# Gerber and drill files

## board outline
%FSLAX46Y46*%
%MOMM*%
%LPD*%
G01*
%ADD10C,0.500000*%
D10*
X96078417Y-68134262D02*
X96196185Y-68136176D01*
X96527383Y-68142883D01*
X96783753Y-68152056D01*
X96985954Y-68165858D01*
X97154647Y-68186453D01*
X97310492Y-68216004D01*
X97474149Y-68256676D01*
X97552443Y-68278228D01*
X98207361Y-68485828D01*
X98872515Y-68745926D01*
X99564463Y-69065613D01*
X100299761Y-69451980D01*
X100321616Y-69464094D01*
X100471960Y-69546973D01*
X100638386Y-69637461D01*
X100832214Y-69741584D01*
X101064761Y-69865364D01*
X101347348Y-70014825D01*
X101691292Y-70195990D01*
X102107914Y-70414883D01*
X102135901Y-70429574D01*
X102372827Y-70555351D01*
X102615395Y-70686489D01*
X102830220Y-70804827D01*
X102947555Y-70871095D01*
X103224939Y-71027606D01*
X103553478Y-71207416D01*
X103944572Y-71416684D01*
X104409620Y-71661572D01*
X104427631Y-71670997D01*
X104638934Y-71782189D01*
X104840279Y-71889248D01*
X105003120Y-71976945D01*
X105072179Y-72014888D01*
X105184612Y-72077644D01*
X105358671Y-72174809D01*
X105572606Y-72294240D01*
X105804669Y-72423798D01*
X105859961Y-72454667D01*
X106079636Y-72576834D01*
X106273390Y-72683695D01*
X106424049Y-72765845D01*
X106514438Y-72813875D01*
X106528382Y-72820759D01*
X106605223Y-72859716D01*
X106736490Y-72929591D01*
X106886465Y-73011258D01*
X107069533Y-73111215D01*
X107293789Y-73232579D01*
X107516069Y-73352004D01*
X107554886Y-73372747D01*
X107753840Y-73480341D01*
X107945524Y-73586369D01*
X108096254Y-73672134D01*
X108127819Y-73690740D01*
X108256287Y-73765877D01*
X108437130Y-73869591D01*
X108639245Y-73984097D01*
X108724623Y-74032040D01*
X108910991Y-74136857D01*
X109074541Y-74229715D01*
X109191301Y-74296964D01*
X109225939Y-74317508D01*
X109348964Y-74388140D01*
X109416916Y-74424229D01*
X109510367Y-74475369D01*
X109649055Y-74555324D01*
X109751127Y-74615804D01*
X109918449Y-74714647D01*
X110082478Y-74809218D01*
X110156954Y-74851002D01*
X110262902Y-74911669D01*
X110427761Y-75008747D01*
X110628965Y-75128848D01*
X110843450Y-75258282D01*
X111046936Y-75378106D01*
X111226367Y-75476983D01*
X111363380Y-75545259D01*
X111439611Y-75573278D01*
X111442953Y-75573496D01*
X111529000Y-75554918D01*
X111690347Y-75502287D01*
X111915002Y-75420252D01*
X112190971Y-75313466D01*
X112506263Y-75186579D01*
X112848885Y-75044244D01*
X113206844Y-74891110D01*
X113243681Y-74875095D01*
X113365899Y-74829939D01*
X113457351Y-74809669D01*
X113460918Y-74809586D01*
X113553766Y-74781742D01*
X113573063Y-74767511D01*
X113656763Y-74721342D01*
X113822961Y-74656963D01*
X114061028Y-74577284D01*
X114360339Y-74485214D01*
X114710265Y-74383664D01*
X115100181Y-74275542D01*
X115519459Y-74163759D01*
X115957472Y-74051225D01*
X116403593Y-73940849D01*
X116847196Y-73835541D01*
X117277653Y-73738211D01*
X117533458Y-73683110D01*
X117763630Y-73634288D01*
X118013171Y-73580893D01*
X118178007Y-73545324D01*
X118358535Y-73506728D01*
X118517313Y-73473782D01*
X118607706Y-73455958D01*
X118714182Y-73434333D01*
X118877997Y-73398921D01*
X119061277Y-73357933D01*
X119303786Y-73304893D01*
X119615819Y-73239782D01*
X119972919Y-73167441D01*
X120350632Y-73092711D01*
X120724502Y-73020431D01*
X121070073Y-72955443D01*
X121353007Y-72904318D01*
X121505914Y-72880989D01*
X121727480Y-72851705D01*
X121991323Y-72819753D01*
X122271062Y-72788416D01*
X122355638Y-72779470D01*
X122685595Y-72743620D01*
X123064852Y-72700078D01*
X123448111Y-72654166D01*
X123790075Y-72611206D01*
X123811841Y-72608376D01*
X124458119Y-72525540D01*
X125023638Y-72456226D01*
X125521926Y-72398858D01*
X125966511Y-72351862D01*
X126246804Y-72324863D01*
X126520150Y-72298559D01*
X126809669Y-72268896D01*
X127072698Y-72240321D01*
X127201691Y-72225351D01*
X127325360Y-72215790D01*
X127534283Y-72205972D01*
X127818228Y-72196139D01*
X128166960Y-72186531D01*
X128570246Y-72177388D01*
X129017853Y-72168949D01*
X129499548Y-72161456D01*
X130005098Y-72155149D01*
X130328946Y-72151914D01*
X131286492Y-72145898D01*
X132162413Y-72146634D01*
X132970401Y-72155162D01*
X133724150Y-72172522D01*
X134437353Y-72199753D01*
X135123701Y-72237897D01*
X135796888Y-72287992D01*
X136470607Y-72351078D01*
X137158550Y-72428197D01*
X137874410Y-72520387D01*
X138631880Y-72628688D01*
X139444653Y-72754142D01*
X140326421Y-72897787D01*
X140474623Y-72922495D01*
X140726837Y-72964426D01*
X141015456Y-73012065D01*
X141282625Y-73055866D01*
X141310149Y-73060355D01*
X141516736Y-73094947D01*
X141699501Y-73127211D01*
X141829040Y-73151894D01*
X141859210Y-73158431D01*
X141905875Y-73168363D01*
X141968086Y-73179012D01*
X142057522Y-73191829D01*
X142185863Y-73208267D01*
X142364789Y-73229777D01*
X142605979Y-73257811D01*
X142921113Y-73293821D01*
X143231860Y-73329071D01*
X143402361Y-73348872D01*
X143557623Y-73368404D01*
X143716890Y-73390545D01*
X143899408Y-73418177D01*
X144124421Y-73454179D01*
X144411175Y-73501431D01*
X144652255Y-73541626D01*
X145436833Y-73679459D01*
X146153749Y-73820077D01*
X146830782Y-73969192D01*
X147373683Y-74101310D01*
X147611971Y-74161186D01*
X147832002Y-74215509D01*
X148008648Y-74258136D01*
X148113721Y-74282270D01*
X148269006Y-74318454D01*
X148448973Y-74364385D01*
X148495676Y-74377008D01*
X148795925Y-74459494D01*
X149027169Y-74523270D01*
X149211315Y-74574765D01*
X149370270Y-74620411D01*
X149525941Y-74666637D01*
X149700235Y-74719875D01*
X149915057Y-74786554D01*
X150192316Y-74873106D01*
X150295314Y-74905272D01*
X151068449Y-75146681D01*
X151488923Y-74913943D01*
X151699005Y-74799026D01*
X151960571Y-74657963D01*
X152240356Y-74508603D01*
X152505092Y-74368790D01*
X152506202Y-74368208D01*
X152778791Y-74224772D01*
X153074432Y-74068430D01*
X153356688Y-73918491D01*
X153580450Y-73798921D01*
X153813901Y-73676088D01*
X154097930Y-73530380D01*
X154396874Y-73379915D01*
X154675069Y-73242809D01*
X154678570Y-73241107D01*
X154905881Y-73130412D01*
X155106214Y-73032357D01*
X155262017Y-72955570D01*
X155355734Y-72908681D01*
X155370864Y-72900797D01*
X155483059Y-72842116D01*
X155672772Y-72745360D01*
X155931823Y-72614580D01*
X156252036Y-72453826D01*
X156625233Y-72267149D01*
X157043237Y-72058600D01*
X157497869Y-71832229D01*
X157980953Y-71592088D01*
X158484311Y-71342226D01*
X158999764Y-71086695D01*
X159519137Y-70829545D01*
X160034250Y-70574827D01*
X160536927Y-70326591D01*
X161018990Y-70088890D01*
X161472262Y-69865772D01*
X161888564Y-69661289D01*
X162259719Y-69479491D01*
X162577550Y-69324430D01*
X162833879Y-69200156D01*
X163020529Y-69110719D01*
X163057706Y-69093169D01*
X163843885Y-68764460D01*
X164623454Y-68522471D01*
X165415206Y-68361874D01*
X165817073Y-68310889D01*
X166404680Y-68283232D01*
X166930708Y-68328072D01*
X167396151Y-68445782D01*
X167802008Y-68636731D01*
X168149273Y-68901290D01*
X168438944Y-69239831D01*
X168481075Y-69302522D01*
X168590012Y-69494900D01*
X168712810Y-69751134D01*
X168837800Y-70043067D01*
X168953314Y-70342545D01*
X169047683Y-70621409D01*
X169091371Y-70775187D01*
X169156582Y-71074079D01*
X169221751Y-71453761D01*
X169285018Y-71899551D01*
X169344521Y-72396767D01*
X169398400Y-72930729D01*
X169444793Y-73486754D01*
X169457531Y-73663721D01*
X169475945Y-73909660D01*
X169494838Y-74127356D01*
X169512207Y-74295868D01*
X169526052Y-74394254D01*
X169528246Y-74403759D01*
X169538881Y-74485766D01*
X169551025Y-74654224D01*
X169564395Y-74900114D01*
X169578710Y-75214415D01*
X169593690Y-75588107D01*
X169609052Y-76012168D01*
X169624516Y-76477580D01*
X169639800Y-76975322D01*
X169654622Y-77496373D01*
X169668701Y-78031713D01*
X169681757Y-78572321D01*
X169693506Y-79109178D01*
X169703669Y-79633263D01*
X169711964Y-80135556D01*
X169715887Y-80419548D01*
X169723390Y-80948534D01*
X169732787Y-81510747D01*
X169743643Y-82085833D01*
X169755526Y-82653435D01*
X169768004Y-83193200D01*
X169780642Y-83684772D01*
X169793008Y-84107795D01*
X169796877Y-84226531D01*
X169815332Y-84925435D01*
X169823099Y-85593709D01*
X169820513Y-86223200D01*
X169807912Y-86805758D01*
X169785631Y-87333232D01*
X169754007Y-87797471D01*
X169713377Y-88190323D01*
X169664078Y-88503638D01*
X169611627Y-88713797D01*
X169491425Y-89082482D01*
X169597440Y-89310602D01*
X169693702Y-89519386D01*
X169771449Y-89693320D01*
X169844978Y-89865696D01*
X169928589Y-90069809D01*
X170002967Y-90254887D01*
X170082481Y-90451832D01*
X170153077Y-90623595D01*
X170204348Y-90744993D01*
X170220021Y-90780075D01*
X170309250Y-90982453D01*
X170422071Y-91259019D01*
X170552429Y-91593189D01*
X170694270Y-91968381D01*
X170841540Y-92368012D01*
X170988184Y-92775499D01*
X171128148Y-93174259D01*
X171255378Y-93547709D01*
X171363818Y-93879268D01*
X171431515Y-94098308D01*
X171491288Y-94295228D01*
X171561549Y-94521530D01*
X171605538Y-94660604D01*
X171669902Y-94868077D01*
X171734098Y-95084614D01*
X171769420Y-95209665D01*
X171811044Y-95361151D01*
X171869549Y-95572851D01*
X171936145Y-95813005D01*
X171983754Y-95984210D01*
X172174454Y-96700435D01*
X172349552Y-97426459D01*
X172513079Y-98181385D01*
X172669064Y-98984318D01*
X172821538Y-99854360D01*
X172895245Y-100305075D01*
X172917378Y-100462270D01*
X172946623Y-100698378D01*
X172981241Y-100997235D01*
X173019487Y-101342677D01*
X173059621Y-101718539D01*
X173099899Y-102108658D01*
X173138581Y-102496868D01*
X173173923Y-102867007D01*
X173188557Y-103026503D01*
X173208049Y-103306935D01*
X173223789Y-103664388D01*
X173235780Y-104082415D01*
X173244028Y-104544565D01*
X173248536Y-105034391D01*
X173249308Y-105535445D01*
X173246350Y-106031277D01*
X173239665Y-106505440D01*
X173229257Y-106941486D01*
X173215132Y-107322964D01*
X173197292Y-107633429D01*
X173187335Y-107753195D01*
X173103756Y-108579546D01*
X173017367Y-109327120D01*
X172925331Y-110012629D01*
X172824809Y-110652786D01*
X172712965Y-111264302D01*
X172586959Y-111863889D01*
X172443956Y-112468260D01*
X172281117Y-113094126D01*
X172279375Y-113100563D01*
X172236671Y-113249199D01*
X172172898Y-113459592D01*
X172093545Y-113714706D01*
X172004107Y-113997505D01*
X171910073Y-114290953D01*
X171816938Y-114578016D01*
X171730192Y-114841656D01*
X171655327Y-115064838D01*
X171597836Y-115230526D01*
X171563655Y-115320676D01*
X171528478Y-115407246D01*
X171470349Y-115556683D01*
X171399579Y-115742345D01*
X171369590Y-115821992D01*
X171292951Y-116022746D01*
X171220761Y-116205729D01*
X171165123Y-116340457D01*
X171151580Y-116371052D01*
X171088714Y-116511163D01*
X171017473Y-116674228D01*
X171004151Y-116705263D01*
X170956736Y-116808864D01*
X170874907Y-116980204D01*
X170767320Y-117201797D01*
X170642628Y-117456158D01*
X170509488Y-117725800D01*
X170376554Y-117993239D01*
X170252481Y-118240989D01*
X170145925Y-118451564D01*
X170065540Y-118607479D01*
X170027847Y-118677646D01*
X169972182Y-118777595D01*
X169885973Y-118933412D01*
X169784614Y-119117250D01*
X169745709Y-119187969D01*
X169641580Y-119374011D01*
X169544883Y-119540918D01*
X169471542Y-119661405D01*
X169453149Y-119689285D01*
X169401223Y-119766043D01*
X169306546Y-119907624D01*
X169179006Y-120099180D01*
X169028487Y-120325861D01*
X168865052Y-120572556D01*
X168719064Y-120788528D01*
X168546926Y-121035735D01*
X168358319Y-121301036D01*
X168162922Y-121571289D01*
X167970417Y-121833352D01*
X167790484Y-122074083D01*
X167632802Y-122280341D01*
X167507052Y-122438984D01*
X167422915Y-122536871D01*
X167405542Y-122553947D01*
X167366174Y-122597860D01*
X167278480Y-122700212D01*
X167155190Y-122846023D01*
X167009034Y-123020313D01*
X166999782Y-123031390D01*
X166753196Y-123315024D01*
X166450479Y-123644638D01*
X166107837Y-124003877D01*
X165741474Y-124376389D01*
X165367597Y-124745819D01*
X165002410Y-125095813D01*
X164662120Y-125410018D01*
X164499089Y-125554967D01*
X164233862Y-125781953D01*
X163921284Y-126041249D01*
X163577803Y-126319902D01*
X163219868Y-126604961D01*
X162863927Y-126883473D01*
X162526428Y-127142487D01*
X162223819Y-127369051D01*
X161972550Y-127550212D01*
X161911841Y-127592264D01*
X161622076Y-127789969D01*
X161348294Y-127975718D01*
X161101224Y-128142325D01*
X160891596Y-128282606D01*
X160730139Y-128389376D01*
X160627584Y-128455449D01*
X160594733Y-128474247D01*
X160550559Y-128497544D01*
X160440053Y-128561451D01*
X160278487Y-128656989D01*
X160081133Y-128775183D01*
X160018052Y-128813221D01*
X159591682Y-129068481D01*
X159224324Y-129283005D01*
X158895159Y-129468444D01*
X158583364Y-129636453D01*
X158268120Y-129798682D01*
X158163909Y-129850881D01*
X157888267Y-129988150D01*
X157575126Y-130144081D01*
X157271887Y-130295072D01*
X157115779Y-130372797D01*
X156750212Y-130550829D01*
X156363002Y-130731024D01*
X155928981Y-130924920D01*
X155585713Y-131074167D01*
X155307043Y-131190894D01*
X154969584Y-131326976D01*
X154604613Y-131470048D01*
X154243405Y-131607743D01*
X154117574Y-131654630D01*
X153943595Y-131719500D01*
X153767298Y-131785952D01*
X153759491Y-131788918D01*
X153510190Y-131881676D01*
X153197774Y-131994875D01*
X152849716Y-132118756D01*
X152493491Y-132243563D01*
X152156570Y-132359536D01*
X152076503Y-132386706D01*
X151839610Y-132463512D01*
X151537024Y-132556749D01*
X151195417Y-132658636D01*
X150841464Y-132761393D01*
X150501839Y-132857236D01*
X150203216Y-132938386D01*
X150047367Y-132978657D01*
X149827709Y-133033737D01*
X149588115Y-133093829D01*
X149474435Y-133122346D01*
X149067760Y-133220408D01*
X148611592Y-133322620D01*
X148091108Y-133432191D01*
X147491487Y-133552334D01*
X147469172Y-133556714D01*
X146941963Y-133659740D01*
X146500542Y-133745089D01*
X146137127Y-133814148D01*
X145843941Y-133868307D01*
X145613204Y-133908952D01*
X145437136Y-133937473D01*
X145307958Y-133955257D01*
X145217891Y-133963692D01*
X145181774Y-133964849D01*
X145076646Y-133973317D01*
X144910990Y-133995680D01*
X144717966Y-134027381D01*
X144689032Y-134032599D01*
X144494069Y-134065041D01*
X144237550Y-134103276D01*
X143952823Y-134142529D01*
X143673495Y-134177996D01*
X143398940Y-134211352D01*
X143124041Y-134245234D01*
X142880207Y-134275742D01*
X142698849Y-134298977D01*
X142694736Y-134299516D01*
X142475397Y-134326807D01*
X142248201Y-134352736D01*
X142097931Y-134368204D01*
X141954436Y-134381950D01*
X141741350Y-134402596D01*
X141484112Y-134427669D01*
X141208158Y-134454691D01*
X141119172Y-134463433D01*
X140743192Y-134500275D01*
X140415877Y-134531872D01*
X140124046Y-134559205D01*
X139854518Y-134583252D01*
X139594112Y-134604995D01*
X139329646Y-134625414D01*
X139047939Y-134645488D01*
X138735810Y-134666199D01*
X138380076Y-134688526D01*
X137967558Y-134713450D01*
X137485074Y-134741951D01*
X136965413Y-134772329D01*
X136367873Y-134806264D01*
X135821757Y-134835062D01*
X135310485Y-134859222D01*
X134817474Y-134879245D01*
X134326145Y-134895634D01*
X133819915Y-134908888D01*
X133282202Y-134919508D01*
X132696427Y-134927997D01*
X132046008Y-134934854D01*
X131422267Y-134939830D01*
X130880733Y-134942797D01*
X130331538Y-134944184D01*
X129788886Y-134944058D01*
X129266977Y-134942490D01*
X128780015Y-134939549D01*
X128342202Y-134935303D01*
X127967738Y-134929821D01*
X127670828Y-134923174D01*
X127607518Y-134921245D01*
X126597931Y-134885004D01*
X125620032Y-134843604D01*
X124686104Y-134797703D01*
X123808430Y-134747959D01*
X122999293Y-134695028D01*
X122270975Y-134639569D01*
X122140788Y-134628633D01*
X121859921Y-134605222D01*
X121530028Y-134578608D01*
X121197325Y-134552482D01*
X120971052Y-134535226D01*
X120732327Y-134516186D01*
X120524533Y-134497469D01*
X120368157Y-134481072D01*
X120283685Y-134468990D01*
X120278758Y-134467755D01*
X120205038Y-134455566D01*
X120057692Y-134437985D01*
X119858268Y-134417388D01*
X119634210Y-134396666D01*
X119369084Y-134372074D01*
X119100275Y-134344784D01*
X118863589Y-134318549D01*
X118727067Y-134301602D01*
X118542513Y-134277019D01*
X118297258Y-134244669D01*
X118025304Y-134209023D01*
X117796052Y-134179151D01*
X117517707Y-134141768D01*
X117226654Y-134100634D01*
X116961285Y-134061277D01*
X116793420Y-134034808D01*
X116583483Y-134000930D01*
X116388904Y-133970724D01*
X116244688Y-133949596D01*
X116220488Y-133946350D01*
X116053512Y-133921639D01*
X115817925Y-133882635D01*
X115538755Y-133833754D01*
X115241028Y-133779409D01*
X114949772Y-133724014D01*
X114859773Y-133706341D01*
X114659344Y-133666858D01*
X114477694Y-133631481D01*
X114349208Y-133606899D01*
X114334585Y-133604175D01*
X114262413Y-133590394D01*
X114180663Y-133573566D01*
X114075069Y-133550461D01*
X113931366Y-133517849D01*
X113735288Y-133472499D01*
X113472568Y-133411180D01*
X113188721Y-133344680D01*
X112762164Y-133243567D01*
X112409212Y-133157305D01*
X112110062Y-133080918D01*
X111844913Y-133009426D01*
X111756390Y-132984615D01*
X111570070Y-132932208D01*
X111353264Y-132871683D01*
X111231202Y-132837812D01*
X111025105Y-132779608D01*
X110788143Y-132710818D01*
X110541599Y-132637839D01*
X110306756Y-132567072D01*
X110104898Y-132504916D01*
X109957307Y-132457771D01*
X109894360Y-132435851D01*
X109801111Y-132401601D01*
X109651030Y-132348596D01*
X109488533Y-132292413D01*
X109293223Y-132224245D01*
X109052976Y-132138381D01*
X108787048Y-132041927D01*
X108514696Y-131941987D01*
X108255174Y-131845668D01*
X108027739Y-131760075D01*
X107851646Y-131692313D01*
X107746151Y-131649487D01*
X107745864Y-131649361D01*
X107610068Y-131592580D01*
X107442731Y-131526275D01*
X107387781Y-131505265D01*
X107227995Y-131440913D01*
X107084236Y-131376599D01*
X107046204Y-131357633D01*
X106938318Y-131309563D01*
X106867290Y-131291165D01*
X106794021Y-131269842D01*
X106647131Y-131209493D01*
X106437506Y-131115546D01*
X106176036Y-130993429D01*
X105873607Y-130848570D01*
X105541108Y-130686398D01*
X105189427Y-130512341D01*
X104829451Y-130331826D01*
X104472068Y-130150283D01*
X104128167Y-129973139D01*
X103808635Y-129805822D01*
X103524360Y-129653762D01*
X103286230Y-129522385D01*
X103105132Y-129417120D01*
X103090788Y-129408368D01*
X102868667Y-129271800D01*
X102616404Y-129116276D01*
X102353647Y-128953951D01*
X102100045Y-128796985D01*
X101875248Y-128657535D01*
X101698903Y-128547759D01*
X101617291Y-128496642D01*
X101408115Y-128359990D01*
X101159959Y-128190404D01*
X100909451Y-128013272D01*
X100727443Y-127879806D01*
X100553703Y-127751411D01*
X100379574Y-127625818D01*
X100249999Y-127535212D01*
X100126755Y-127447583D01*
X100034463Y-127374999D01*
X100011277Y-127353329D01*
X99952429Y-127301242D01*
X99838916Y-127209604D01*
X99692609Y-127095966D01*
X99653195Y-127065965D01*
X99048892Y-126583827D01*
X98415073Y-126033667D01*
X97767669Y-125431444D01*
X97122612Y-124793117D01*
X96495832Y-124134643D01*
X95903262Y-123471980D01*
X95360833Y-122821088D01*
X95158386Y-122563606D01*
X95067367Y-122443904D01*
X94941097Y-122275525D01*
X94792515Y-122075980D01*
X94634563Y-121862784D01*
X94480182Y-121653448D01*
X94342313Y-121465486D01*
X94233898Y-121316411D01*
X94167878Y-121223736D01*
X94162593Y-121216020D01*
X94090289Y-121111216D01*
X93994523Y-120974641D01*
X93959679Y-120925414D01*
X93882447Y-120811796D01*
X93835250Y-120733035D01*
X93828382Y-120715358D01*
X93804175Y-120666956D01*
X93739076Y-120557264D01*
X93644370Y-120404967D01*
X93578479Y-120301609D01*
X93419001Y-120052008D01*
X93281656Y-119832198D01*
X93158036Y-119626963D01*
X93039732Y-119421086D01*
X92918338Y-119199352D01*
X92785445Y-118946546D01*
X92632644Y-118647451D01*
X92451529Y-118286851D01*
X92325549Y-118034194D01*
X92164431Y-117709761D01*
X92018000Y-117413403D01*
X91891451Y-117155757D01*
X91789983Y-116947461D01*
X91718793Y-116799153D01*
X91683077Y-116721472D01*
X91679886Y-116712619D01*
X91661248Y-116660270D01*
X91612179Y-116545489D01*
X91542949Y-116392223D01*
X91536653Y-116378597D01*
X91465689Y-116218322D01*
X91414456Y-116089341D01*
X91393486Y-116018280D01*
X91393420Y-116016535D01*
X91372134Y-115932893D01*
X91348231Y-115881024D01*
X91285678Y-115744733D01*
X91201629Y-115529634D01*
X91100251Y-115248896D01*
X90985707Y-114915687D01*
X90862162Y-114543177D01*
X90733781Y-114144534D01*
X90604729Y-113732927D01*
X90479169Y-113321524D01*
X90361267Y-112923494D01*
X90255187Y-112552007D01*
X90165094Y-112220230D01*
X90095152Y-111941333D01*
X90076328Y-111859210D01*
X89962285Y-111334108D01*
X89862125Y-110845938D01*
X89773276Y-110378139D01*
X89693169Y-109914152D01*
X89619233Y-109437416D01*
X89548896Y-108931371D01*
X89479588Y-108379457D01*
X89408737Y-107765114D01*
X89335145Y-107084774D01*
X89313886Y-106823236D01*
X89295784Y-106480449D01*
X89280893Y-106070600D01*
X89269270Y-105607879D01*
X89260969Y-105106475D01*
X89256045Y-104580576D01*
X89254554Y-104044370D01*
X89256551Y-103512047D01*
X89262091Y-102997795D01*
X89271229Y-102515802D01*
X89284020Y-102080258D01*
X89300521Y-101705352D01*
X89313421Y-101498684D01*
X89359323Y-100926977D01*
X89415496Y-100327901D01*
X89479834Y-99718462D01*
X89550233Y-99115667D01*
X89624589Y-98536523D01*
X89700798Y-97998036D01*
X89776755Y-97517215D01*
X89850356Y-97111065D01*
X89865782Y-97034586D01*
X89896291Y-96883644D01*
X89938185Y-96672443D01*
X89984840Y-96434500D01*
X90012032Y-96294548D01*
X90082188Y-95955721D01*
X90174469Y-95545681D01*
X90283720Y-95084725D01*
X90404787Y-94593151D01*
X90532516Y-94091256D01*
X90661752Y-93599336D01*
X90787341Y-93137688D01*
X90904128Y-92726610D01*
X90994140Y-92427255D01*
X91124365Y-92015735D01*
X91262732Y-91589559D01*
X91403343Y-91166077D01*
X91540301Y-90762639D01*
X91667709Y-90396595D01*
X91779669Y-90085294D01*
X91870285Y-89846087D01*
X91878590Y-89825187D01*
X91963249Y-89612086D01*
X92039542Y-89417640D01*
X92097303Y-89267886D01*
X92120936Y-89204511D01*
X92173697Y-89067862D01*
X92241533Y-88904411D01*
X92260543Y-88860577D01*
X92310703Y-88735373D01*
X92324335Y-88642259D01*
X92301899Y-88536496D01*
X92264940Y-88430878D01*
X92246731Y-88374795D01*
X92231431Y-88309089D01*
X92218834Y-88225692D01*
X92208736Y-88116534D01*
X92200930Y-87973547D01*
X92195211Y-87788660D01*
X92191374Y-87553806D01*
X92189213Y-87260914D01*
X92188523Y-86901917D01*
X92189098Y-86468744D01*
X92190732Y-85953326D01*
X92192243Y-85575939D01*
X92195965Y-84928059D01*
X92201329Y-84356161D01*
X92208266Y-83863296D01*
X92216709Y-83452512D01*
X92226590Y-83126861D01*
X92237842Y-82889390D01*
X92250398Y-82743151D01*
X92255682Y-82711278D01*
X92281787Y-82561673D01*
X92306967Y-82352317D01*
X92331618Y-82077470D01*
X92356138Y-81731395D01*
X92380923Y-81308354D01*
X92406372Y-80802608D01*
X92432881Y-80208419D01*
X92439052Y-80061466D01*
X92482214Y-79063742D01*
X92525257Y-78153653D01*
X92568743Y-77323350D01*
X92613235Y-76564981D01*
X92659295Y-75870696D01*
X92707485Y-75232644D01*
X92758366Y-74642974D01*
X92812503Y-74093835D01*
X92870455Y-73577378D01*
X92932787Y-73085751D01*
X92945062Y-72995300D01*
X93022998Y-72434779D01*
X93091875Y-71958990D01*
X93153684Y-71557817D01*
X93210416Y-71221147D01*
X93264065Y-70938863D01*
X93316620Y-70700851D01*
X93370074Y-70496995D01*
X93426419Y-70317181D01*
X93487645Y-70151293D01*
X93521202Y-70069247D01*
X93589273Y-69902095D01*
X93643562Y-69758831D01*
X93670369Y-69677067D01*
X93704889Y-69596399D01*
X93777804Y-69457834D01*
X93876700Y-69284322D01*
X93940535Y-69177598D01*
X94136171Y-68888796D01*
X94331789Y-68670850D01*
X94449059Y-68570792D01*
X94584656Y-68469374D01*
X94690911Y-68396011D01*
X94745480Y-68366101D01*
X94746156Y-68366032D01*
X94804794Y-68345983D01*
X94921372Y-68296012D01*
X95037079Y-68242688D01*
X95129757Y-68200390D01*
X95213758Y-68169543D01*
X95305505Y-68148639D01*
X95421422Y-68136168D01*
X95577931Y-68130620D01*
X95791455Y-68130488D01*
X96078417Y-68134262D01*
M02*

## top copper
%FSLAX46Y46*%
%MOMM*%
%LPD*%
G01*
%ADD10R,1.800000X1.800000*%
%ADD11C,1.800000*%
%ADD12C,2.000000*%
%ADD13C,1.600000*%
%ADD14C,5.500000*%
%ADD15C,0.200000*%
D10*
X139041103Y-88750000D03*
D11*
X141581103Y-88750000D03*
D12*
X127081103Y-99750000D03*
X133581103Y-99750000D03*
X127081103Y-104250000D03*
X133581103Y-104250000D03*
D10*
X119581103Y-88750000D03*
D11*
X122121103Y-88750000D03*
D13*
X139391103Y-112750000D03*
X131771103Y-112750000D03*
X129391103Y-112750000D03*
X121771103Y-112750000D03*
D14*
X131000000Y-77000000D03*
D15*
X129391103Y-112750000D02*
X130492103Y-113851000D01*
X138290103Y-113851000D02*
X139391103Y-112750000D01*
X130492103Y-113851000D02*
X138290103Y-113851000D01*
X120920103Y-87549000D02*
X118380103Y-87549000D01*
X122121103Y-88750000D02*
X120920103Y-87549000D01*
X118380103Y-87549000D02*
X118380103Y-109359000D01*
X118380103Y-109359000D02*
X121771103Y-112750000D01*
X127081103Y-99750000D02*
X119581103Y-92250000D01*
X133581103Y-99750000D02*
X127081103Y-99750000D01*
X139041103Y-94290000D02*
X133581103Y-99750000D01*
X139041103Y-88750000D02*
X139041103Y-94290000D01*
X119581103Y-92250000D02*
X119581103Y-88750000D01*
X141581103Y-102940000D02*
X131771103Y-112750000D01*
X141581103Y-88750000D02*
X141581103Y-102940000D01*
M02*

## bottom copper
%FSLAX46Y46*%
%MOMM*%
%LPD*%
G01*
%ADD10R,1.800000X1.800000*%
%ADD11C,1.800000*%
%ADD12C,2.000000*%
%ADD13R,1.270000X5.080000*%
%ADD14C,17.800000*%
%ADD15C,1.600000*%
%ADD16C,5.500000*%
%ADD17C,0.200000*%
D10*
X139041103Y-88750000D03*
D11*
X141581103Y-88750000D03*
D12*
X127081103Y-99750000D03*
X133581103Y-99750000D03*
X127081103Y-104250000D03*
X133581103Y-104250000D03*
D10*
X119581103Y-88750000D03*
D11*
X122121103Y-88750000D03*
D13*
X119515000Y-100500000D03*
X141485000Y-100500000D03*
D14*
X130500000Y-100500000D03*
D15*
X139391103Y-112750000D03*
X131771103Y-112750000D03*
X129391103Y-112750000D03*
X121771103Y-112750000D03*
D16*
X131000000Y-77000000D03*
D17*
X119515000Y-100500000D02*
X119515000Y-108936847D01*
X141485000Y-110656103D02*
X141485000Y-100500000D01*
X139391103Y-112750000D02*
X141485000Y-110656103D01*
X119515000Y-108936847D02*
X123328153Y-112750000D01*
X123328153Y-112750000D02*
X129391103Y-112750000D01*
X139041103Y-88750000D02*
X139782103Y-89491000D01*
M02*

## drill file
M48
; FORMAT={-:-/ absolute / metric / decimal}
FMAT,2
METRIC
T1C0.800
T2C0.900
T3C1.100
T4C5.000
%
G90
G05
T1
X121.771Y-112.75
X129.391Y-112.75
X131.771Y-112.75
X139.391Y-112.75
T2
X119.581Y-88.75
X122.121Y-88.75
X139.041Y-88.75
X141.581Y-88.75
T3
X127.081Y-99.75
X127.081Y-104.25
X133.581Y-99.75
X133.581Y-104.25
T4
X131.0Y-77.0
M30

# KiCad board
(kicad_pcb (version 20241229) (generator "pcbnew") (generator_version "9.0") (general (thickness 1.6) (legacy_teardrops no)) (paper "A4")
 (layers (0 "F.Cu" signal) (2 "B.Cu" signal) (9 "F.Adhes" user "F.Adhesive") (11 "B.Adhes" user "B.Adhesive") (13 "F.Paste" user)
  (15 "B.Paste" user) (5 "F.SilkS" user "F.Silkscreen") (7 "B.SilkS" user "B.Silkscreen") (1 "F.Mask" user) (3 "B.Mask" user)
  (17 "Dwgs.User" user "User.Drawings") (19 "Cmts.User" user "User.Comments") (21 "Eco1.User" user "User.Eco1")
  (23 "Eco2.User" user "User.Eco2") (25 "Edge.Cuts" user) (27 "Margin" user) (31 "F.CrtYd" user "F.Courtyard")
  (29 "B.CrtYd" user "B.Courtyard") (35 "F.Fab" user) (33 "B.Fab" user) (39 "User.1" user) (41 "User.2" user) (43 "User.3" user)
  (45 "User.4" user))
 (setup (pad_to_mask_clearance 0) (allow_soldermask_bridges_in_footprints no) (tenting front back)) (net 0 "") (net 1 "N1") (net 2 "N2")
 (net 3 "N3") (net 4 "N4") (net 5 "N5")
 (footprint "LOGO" (layer "F.Cu") (at 100 77 10)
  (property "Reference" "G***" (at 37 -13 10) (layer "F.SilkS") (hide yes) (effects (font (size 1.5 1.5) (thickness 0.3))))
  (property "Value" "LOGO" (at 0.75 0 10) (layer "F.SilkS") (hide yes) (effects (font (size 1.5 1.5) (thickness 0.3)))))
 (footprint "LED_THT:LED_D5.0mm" (layer "F.Cu") (at 139.041103 88.75)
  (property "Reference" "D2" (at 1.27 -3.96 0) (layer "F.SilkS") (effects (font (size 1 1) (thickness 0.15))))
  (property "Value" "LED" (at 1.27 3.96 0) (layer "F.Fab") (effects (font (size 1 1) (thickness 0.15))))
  (pad "1" thru_hole rect (at 0 0) (size 1.8 1.8) (drill 0.9) (layers "*.Cu" "*.Mask") (remove_unused_layers no) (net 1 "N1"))
  (pad "2" thru_hole circle (at 2.54 0) (size 1.8 1.8) (drill 0.9) (layers "*.Cu" "*.Mask") (remove_unused_layers no) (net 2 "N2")))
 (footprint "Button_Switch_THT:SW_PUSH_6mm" (layer "F.Cu") (at 127.081103 99.75)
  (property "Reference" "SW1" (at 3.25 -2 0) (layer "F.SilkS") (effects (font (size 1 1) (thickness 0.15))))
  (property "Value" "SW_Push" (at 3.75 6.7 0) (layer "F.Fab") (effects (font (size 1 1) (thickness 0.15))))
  (pad "1" thru_hole circle (at 0 0 90) (size 2 2) (drill 1.1) (layers "*.Cu" "*.Mask") (remove_unused_layers no) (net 1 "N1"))
  (pad "1" thru_hole circle (at 6.5 0 90) (size 2 2) (drill 1.1) (layers "*.Cu" "*.Mask") (remove_unused_layers no) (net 1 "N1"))
  (pad "2" thru_hole circle (at 0 4.5 90) (size 2 2) (drill 1.1) (layers "*.Cu" "*.Mask") (remove_unused_layers no) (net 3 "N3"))
  (pad "2" thru_hole circle (at 6.5 4.5 90) (size 2 2) (drill 1.1) (layers "*.Cu" "*.Mask") (remove_unused_layers no) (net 3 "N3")))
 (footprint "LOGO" (layer "F.Cu") (at 132 102)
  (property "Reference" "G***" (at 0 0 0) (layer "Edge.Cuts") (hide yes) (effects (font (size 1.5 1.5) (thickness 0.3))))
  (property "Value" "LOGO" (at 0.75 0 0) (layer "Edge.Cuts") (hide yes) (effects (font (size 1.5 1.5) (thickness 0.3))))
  (fp_poly
   (pts (xy -35.921583 -33.865738) (xy -35.803815 -33.863824) (xy -35.472617 -33.857117) (xy -35.216247 -33.847944)
    (xy -35.014046 -33.834142) (xy -34.845353 -33.813547) (xy -34.689508 -33.783996) (xy -34.525851 -33.743324) (xy -34.447557 -33.721772)
    (xy -33.792639 -33.514172) (xy -33.127485 -33.254074) (xy -32.435537 -32.934387) (xy -31.700239 -32.54802) (xy -31.678384 -32.535906)
    (xy -31.52804 -32.453027) (xy -31.361614 -32.362539) (xy -31.167786 -32.258416) (xy -30.935239 -32.134636) (xy -30.652652 -31.985175)
    (xy -30.308708 -31.80401) (xy -29.892086 -31.585117) (xy -29.864099 -31.570426) (xy -29.627173 -31.444649) (xy -29.384605 -31.313511)
    (xy -29.16978 -31.195173) (xy -29.052445 -31.128905) (xy -28.775061 -30.972394) (xy -28.446522 -30.792584) (xy -28.055428 -30.583316)
    (xy -27.59038 -30.338428) (xy -27.572369 -30.329003) (xy -27.361066 -30.217811) (xy -27.159721 -30.110752) (xy -26.99688 -30.023055)
    (xy -26.927821 -29.985112) (xy -26.815388 -29.922356) (xy -26.641329 -29.825191) (xy -26.427394 -29.70576) (xy -26.195331 -29.576202)
    (xy -26.140039 -29.545333) (xy -25.920364 -29.423166) (xy -25.72661 -29.316305) (xy -25.575951 -29.234155) (xy -25.485562 -29.186125)
    (xy -25.471618 -29.179241) (xy -25.394777 -29.140284) (xy -25.26351 -29.070409) (xy -25.113535 -28.988742) (xy -24.930467 -28.888785)
    (xy -24.706211 -28.767421) (xy -24.483931 -28.647996) (xy -24.445114 -28.627253) (xy -24.24616 -28.519659) (xy -24.054476 -28.413631)
    (xy -23.903746 -28.327866) (xy -23.872181 -28.30926) (xy -23.743713 -28.234123) (xy -23.56287 -28.130409) (xy -23.360755 -28.015903)
    (xy -23.275377 -27.96796) (xy -23.089009 -27.863143) (xy -22.925459 -27.770285) (xy -22.808699 -27.703036) (xy -22.774061 -27.682492)
    (xy -22.651036 -27.61186) (xy -22.583084 -27.575771) (xy -22.489633 -27.524631) (xy -22.350945 -27.444676) (xy -22.248873 -27.384196)
    (xy -22.081551 -27.285353) (xy -21.917522 -27.190782) (xy -21.843046 -27.148998) (xy -21.737098 -27.088331) (xy -21.572239 -26.991253)
    (xy -21.371035 -26.871152) (xy -21.15655 -26.741718) (xy -20.953064 -26.621894) (xy -20.773633 -26.523017) (xy -20.63662 -26.454741)
    (xy -20.560389 -26.426722) (xy -20.557047 -26.426504) (xy -20.471 -26.445082) (xy -20.309653 -26.497713) (xy -20.084998 -26.579748)
    (xy -19.809029 -26.686534) (xy -19.493737 -26.813421) (xy -19.151115 -26.955756) (xy -18.793156 -27.10889) (xy -18.756319 -27.124905)
    (xy -18.634101 -27.170061) (xy -18.542649 -27.190331) (xy -18.539082 -27.190414) (xy -18.446234 -27.218258) (xy -18.426937 -27.232489)
    (xy -18.343237 -27.278658) (xy -18.177039 -27.343037) (xy -17.938972 -27.422716) (xy -17.639661 -27.514786) (xy -17.289735 -27.616336)
    (xy -16.899819 -27.724458) (xy -16.480541 -27.836241) (xy -16.042528 -27.948775) (xy -15.596407 -28.059151) (xy -15.152804 -28.164459)
    (xy -14.722347 -28.261789) (xy -14.466542 -28.31689) (xy -14.23637 -28.365712) (xy -13.986829 -28.419107) (xy -13.821993 -28.454676)
    (xy -13.641465 -28.493272) (xy -13.482687 -28.526218) (xy -13.392294 -28.544042) (xy -13.285818 -28.565667) (xy -13.122003 -28.601079)
    (xy -12.938723 -28.642067) (xy -12.696214 -28.695107) (xy -12.384181 -28.760218) (xy -12.027081 -28.832559) (xy -11.649368 -28.907289)
    (xy -11.275498 -28.979569) (xy -10.929927 -29.044557) (xy -10.646993 -29.095682) (xy -10.494086 -29.119011) (xy -10.27252 -29.148295)
    (xy -10.008677 -29.180247) (xy -9.728938 -29.211584) (xy -9.644362 -29.22053) (xy -9.314405 -29.25638) (xy -8.935148 -29.299922)
    (xy -8.551889 -29.345834) (xy -8.209925 -29.388794) (xy -8.188159 -29.391624) (xy -7.541881 -29.47446) (xy -6.976362 -29.543774)
    (xy -6.478074 -29.601142) (xy -6.033489 -29.648138) (xy -5.753196 -29.675137) (xy -5.47985 -29.701441) (xy -5.190331 -29.731104)
    (xy -4.927302 -29.759679) (xy -4.798309 -29.774649) (xy -4.67464 -29.78421) (xy -4.465717 -29.794028) (xy -4.181772 -29.803861)
    (xy -3.83304 -29.813469) (xy -3.429754 -29.822612) (xy -2.982147 -29.831051) (xy -2.500452 -29.838544) (xy -1.994902 -29.844851)
    (xy -1.671054 -29.848086) (xy -0.713508 -29.854102) (xy 0.162413 -29.853366) (xy 0.970401 -29.844838) (xy 1.72415 -29.827478)
    (xy 2.437353 -29.800247) (xy 3.123701 -29.762103) (xy 3.796888 -29.712008) (xy 4.470607 -29.648922) (xy 5.15855 -29.571803)
    (xy 5.87441 -29.479613) (xy 6.63188 -29.371312) (xy 7.444653 -29.245858) (xy 8.326421 -29.102213) (xy 8.474623 -29.077505)
    (xy 8.726837 -29.035574) (xy 9.015456 -28.987935) (xy 9.282625 -28.944134) (xy 9.310149 -28.939645) (xy 9.516736 -28.905053)
    (xy 9.699501 -28.872789) (xy 9.82904 -28.848106) (xy 9.85921 -28.841569) (xy 9.905875 -28.831637) (xy 9.968086 -28.820988)
    (xy 10.057522 -28.808171) (xy 10.185863 -28.791733) (xy 10.364789 -28.770223) (xy 10.605979 -28.742189) (xy 10.921113 -28.706179)
    (xy 11.23186 -28.670929) (xy 11.402361 -28.651128) (xy 11.557623 -28.631596) (xy 11.71689 -28.609455) (xy 11.899408 -28.581823)
    (xy 12.124421 -28.545821) (xy 12.411175 -28.498569) (xy 12.652255 -28.458374) (xy 13.436833 -28.320541) (xy 14.153749 -28.179923)
    (xy 14.830782 -28.030808) (xy 15.373683 -27.89869) (xy 15.611971 -27.838814) (xy 15.832002 -27.784491) (xy 16.008648 -27.741864)
    (xy 16.113721 -27.71773) (xy 16.269006 -27.681546) (xy 16.448973 -27.635615) (xy 16.495676 -27.622992) (xy 16.795925 -27.540506)
    (xy 17.027169 -27.47673) (xy 17.211315 -27.425235) (xy 17.37027 -27.379589) (xy 17.525941 -27.333363) (xy 17.700235 -27.280125)
    (xy 17.915057 -27.213446) (xy 18.192316 -27.126894) (xy 18.295314 -27.094728) (xy 19.068449 -26.853319) (xy 19.488923 -27.086057)
    (xy 19.699005 -27.200974) (xy 19.960571 -27.342037) (xy 20.240356 -27.491397) (xy 20.505092 -27.63121) (xy 20.506202 -27.631792)
    (xy 20.778791 -27.775228) (xy 21.074432 -27.93157) (xy 21.356688 -28.081509) (xy 21.58045 -28.201079) (xy 21.813901 -28.323912)
    (xy 22.09793 -28.46962) (xy 22.396874 -28.620085) (xy 22.675069 -28.757191) (xy 22.67857 -28.758893) (xy 22.905881 -28.869588)
    (xy 23.106214 -28.967643) (xy 23.262017 -29.04443) (xy 23.355734 -29.091319) (xy 23.370864 -29.099203) (xy 23.483059 -29.157884)
    (xy 23.672772 -29.25464) (xy 23.931823 -29.38542) (xy 24.252036 -29.546174) (xy 24.625233 -29.732851) (xy 25.043237 -29.9414)
    (xy 25.497869 -30.167771) (xy 25.980953 -30.407912) (xy 26.484311 -30.657774) (xy 26.999764 -30.913305) (xy 27.519137 -31.170455)
    (xy 28.03425 -31.425173) (xy 28.536927 -31.673409) (xy 29.01899 -31.91111) (xy 29.472262 -32.134228) (xy 29.888564 -32.338711)
    (xy 30.259719 -32.520509) (xy 30.57755 -32.67557) (xy 30.833879 -32.799844) (xy 31.020529 -32.889281) (xy 31.057706 -32.906831)
    (xy 31.843885 -33.23554) (xy 32.623454 -33.477529) (xy 33.415206 -33.638126) (xy 33.817073 -33.689111) (xy 34.40468 -33.716768)
    (xy 34.930708 -33.671928) (xy 35.396151 -33.554218) (xy 35.802008 -33.363269) (xy 36.149273 -33.09871) (xy 36.438944 -32.760169)
    (xy 36.481075 -32.697478) (xy 36.590012 -32.5051) (xy 36.71281 -32.248866) (xy 36.8378 -31.956933) (xy 36.953314 -31.657455)
    (xy 37.047683 -31.378591) (xy 37.091371 -31.224813) (xy 37.156582 -30.925921) (xy 37.221751 -30.546239) (xy 37.285018 -30.100449)
    (xy 37.344521 -29.603233) (xy 37.3984 -29.069271) (xy 37.444793 -28.513246) (xy 37.457531 -28.336279) (xy 37.475945 -28.09034)
    (xy 37.494838 -27.872644) (xy 37.512207 -27.704132) (xy 37.526052 -27.605746) (xy 37.528246 -27.596241) (xy 37.538881 -27.514234)
    (xy 37.551025 -27.345776) (xy 37.564395 -27.099886) (xy 37.57871 -26.785585) (xy 37.59369 -26.411893) (xy 37.609052 -25.987832)
    (xy 37.624516 -25.52242) (xy 37.6398 -25.024678) (xy 37.654622 -24.503627) (xy 37.668701 -23.968287) (xy 37.681757 -23.427679)
    (xy 37.693506 -22.890822) (xy 37.703669 -22.366737) (xy 37.711964 -21.864444) (xy 37.715887 -21.580452) (xy 37.72339 -21.051466)
    (xy 37.732787 -20.489253) (xy 37.743643 -19.914167) (xy 37.755526 -19.346565) (xy 37.768004 -18.8068) (xy 37.780642 -18.315228)
    (xy 37.793008 -17.892205) (xy 37.796877 -17.773469) (xy 37.815332 -17.074565) (xy 37.823099 -16.406291) (xy 37.820513 -15.7768)
    (xy 37.807912 -15.194242) (xy 37.785631 -14.666768) (xy 37.754007 -14.202529) (xy 37.713377 -13.809677) (xy 37.664078 -13.496362)
    (xy 37.611627 -13.286203) (xy 37.491425 -12.917518) (xy 37.59744 -12.689398) (xy 37.693702 -12.480614) (xy 37.771449 -12.30668)
    (xy 37.844978 -12.134304) (xy 37.928589 -11.930191) (xy 38.002967 -11.745113) (xy 38.082481 -11.548168) (xy 38.153077 -11.376405)
    (xy 38.204348 -11.255007) (xy 38.220021 -11.219925) (xy 38.30925 -11.017547) (xy 38.422071 -10.740981) (xy 38.552429 -10.406811)
    (xy 38.69427 -10.031619) (xy 38.84154 -9.631988) (xy 38.988184 -9.224501) (xy 39.128148 -8.825741) (xy 39.255378 -8.452291)
    (xy 39.363818 -8.120732) (xy 39.431515 -7.901692) (xy 39.491288 -7.704772) (xy 39.561549 -7.47847) (xy 39.605538 -7.339396)
    (xy 39.669902 -7.131923) (xy 39.734098 -6.915386) (xy 39.76942 -6.790335) (xy 39.811044 -6.638849) (xy 39.869549 -6.427149)
    (xy 39.936145 -6.186995) (xy 39.983754 -6.01579) (xy 40.174454 -5.299565) (xy 40.349552 -4.573541) (xy 40.513079 -3.818615)
    (xy 40.669064 -3.015682) (xy 40.821538 -2.14564) (xy 40.895245 -1.694925) (xy 40.917378 -1.53773) (xy 40.946623 -1.301622)
    (xy 40.981241 -1.002765) (xy 41.019487 -0.657323) (xy 41.059621 -0.281461) (xy 41.099899 0.108658) (xy 41.138581 0.496868)
    (xy 41.173923 0.867007) (xy 41.188557 1.026503) (xy 41.208049 1.306935) (xy 41.223789 1.664388) (xy 41.23578 2.082415)
    (xy 41.244028 2.544565) (xy 41.248536 3.034391) (xy 41.249308 3.535445) (xy 41.24635 4.031277) (xy 41.239665 4.50544)
    (xy 41.229257 4.941486) (xy 41.215132 5.322964) (xy 41.197292 5.633429) (xy 41.187335 5.753195) (xy 41.103756 6.579546)
    (xy 41.017367 7.32712) (xy 40.925331 8.012629) (xy 40.824809 8.652786) (xy 40.712965 9.264302) (xy 40.586959 9.863889)
    (xy 40.443956 10.46826) (xy 40.281117 11.094126) (xy 40.279375 11.100563) (xy 40.236671 11.249199) (xy 40.172898 11.459592)
    (xy 40.093545 11.714706) (xy 40.004107 11.997505) (xy 39.910073 12.290953) (xy 39.816938 12.578016) (xy 39.730192 12.841656)
    (xy 39.655327 13.064838) (xy 39.597836 13.230526) (xy 39.563655 13.320676) (xy 39.528478 13.407246) (xy 39.470349 13.556683)
    (xy 39.399579 13.742345) (xy 39.36959 13.821992) (xy 39.292951 14.022746) (xy 39.220761 14.205729) (xy 39.165123 14.340457)
    (xy 39.15158 14.371052) (xy 39.088714 14.511163) (xy 39.017473 14.674228) (xy 39.004151 14.705263) (xy 38.956736 14.808864)
    (xy 38.874907 14.980204) (xy 38.76732 15.201797) (xy 38.642628 15.456158) (xy 38.509488 15.7258) (xy 38.376554 15.993239)
    (xy 38.252481 16.240989) (xy 38.145925 16.451564) (xy 38.06554 16.607479) (xy 38.027847 16.677646) (xy 37.972182 16.777595)
    (xy 37.885973 16.933412) (xy 37.784614 17.11725) (xy 37.745709 17.187969) (xy 37.64158 17.374011) (xy 37.544883 17.540918)
    (xy 37.471542 17.661405) (xy 37.453149 17.689285) (xy 37.401223 17.766043) (xy 37.306546 17.907624) (xy 37.179006 18.09918)
    (xy 37.028487 18.325861) (xy 36.865052 18.572556) (xy 36.719064 18.788528) (xy 36.546926 19.035735) (xy 36.358319 19.301036)
    (xy 36.162922 19.571289) (xy 35.970417 19.833352) (xy 35.790484 20.074083) (xy 35.632802 20.280341) (xy 35.507052 20.438984)
    (xy 35.422915 20.536871) (xy 35.405542 20.553947) (xy 35.366174 20.59786) (xy 35.27848 20.700212) (xy 35.15519 20.846023)
    (xy 35.009034 21.020313) (xy 34.999782 21.03139) (xy 34.753196 21.315024) (xy 34.450479 21.644638) (xy 34.107837 22.003877)
    (xy 33.741474 22.376389) (xy 33.367597 22.745819) (xy 33.00241 23.095813) (xy 32.66212 23.410018) (xy 32.499089 23.554967)
    (xy 32.233862 23.781953) (xy 31.921284 24.041249) (xy 31.577803 24.319902) (xy 31.219868 24.604961) (xy 30.863927 24.883473)
    (xy 30.526428 25.142487) (xy 30.223819 25.369051) (xy 29.97255 25.550212) (xy 29.911841 25.592264) (xy 29.622076 25.789969)
    (xy 29.348294 25.975718) (xy 29.101224 26.142325) (xy 28.891596 26.282606) (xy 28.730139 26.389376) (xy 28.627584 26.455449)
    (xy 28.594733 26.474247) (xy 28.550559 26.497544) (xy 28.440053 26.561451) (xy 28.278487 26.656989) (xy 28.081133 26.775183)
    (xy 28.018052 26.813221) (xy 27.591682 27.068481) (xy 27.224324 27.283005) (xy 26.895159 27.468444) (xy 26.583364 27.636453)
    (xy 26.26812 27.798682) (xy 26.163909 27.850881) (xy 25.888267 27.98815) (xy 25.575126 28.144081) (xy 25.271887 28.295072)
    (xy 25.115779 28.372797) (xy 24.750212 28.550829) (xy 24.363002 28.731024) (xy 23.928981 28.92492) (xy 23.585713 29.074167)
    (xy 23.307043 29.190894) (xy 22.969584 29.326976) (xy 22.604613 29.470048) (xy 22.243405 29.607743) (xy 22.117574 29.65463)
    (xy 21.943595 29.7195) (xy 21.767298 29.785952) (xy 21.759491 29.788918) (xy 21.51019 29.881676) (xy 21.197774 29.994875)
    (xy 20.849716 30.118756) (xy 20.493491 30.243563) (xy 20.15657 30.359536) (xy 20.076503 30.386706) (xy 19.83961 30.463512)
    (xy 19.537024 30.556749) (xy 19.195417 30.658636) (xy 18.841464 30.761393) (xy 18.501839 30.857236) (xy 18.203216 30.938386)
    (xy 18.047367 30.978657) (xy 17.827709 31.033737) (xy 17.588115 31.093829) (xy 17.474435 31.122346) (xy 17.06776 31.220408)
    (xy 16.611592 31.32262) (xy 16.091108 31.432191) (xy 15.491487 31.552334) (xy 15.469172 31.556714) (xy 14.941963 31.65974)
    (xy 14.500542 31.745089) (xy 14.137127 31.814148) (xy 13.843941 31.868307) (xy 13.613204 31.908952) (xy 13.437136 31.937473)
    (xy 13.307958 31.955257) (xy 13.217891 31.963692) (xy 13.181774 31.964849) (xy 13.076646 31.973317) (xy 12.91099 31.99568)
    (xy 12.717966 32.027381) (xy 12.689032 32.032599) (xy 12.494069 32.065041) (xy 12.23755 32.103276) (xy 11.952823 32.142529)
    (xy 11.673495 32.177996) (xy 11.39894 32.211352) (xy 11.124041 32.245234) (xy 10.880207 32.275742) (xy 10.698849 32.298977)
    (xy 10.694736 32.299516) (xy 10.475397 32.326807) (xy 10.248201 32.352736) (xy 10.097931 32.368204) (xy 9.954436 32.38195)
    (xy 9.74135 32.402596) (xy 9.484112 32.427669) (xy 9.208158 32.454691) (xy 9.119172 32.463433) (xy 8.743192 32.500275)
    (xy 8.415877 32.531872) (xy 8.124046 32.559205) (xy 7.854518 32.583252) (xy 7.594112 32.604995) (xy 7.329646 32.625414)
    (xy 7.047939 32.645488) (xy 6.73581 32.666199) (xy 6.380076 32.688526) (xy 5.967558 32.71345) (xy 5.485074 32.741951)
    (xy 4.965413 32.772329) (xy 4.367873 32.806264) (xy 3.821757 32.835062) (xy 3.310485 32.859222) (xy 2.817474 32.879245)
    (xy 2.326145 32.895634) (xy 1.819915 32.908888) (xy 1.282202 32.919508) (xy 0.696427 32.927997) (xy 0.046008 32.934854)
    (xy -0.577733 32.93983) (xy -1.119267 32.942797) (xy -1.668462 32.944184) (xy -2.211114 32.944058) (xy -2.733023 32.94249)
    (xy -3.219985 32.939549) (xy -3.657798 32.935303) (xy -4.032262 32.929821) (xy -4.329172 32.923174) (xy -4.392482 32.921245)
    (xy -5.402069 32.885004) (xy -6.379968 32.843604) (xy -7.313896 32.797703) (xy -8.19157 32.747959) (xy -9.000707 32.695028)
    (xy -9.729025 32.639569) (xy -9.859212 32.628633) (xy -10.140079 32.605222) (xy -10.469972 32.578608) (xy -10.802675 32.552482)
    (xy -11.028948 32.535226) (xy -11.267673 32.516186) (xy -11.475467 32.497469) (xy -11.631843 32.481072) (xy -11.716315 32.46899)
    (xy -11.721242 32.467755) (xy -11.794962 32.455566) (xy -11.942308 32.437985) (xy -12.141732 32.417388) (xy -12.36579 32.396666)
    (xy -12.630916 32.372074) (xy -12.899725 32.344784) (xy -13.136411 32.318549) (xy -13.272933 32.301602) (xy -13.457487 32.277019)
    (xy -13.702742 32.244669) (xy -13.974696 32.209023) (xy -14.203948 32.179151) (xy -14.482293 32.141768) (xy -14.773346 32.100634)
    (xy -15.038715 32.061277) (xy -15.20658 32.034808) (xy -15.416517 32.00093) (xy -15.611096 31.970724) (xy -15.755312 31.949596)
    (xy -15.779512 31.94635) (xy -15.946488 31.921639) (xy -16.182075 31.882635) (xy -16.461245 31.833754) (xy -16.758972 31.779409)
    (xy -17.050228 31.724014) (xy -17.140227 31.706341) (xy -17.340656 31.666858) (xy -17.522306 31.631481) (xy -17.650792 31.606899)
    (xy -17.665415 31.604175) (xy -17.737587 31.590394) (xy -17.819337 31.573566) (xy -17.924931 31.550461) (xy -18.068634 31.517849)
    (xy -18.264712 31.472499) (xy -18.527432 31.41118) (xy -18.811279 31.34468) (xy -19.237836 31.243567) (xy -19.590788 31.157305)
    (xy -19.889938 31.080918) (xy -20.155087 31.009426) (xy -20.24361 30.984615) (xy -20.42993 30.932208) (xy -20.646736 30.871683)
    (xy -20.768798 30.837812) (xy -20.974895 30.779608) (xy -21.211857 30.710818) (xy -21.458401 30.637839) (xy -21.693244 30.567072)
    (xy -21.895102 30.504916) (xy -22.042693 30.457771) (xy -22.10564 30.435851) (xy -22.198889 30.401601) (xy -22.34897 30.348596)
    (xy -22.511467 30.292413) (xy -22.706777 30.224245) (xy -22.947024 30.138381) (xy -23.212952 30.041927) (xy -23.485304 29.941987)
    (xy -23.744826 29.845668) (xy -23.972261 29.760075) (xy -24.148354 29.692313) (xy -24.253849 29.649487) (xy -24.254136 29.649361)
    (xy -24.389932 29.59258) (xy -24.557269 29.526275) (xy -24.612219 29.505265) (xy -24.772005 29.440913) (xy -24.915764 29.376599)
    (xy -24.953796 29.357633) (xy -25.061682 29.309563) (xy -25.13271 29.291165) (xy -25.205979 29.269842) (xy -25.352869 29.209493)
    (xy -25.562494 29.115546) (xy -25.823964 28.993429) (xy -26.126393 28.84857) (xy -26.458892 28.686398) (xy -26.810573 28.512341)
    (xy -27.170549 28.331826) (xy -27.527932 28.150283) (xy -27.871833 27.973139) (xy -28.191365 27.805822) (xy -28.47564 27.653762)
    (xy -28.71377 27.522385) (xy -28.894868 27.41712) (xy -28.909212 27.408368) (xy -29.131333 27.2718) (xy -29.383596 27.116276)
    (xy -29.646353 26.953951) (xy -29.899955 26.796985) (xy -30.124752 26.657535) (xy -30.301097 26.547759) (xy -30.382709 26.496642)
    (xy -30.591885 26.35999) (xy -30.840041 26.190404) (xy -31.090549 26.013272) (xy -31.272557 25.879806) (xy -31.446297 25.751411)
    (xy -31.620426 25.625818) (xy -31.750001 25.535212) (xy -31.873245 25.447583) (xy -31.965537 25.374999) (xy -31.988723 25.353329)
    (xy -32.047571 25.301242) (xy -32.161084 25.209604) (xy -32.307391 25.095966) (xy -32.346805 25.065965) (xy -32.951108 24.583827)
    (xy -33.584927 24.033667) (xy -34.232331 23.431444) (xy -34.877388 22.793117) (xy -35.504168 22.134643) (xy -36.096738 21.47198)
    (xy -36.639167 20.821088) (xy -36.841614 20.563606) (xy -36.932633 20.443904) (xy -37.058903 20.275525) (xy -37.207485 20.07598)
    (xy -37.365437 19.862784) (xy -37.519818 19.653448) (xy -37.657687 19.465486) (xy -37.766102 19.316411) (xy -37.832122 19.223736)
    (xy -37.837407 19.21602) (xy -37.909711 19.111216) (xy -38.005477 18.974641) (xy -38.040321 18.925414) (xy -38.117553 18.811796)
    (xy -38.16475 18.733035) (xy -38.171618 18.715358) (xy -38.195825 18.666956) (xy -38.260924 18.557264) (xy -38.35563 18.404967)
    (xy -38.421521 18.301609) (xy -38.580999 18.052008) (xy -38.718344 17.832198) (xy -38.841964 17.626963) (xy -38.960268 17.421086)
    (xy -39.081662 17.199352) (xy -39.214555 16.946546) (xy -39.367356 16.647451) (xy -39.548471 16.286851) (xy -39.674451 16.034194)
    (xy -39.835569 15.709761) (xy -39.982 15.413403) (xy -40.108549 15.155757) (xy -40.210017 14.947461) (xy -40.281207 14.799153)
    (xy -40.316923 14.721472) (xy -40.320114 14.712619) (xy -40.338752 14.66027) (xy -40.387821 14.545489) (xy -40.457051 14.392223)
    (xy -40.463347 14.378597) (xy -40.534311 14.218322) (xy -40.585544 14.089341) (xy -40.606514 14.01828) (xy -40.60658 14.016535)
    (xy -40.627866 13.932893) (xy -40.651769 13.881024) (xy -40.714322 13.744733) (xy -40.798371 13.529634) (xy -40.899749 13.248896)
    (xy -41.014293 12.915687) (xy -41.137838 12.543177) (xy -41.266219 12.144534) (xy -41.395271 11.732927) (xy -41.520831 11.321524)
    (xy -41.638733 10.923494) (xy -41.744813 10.552007) (xy -41.834906 10.22023) (xy -41.904848 9.941333) (xy -41.923672 9.85921)
    (xy -42.037715 9.334108) (xy -42.137875 8.845938) (xy -42.226724 8.378139) (xy -42.306831 7.914152) (xy -42.380767 7.437416)
    (xy -42.451104 6.931371) (xy -42.520412 6.379457) (xy -42.591263 5.765114) (xy -42.664855 5.084774) (xy -42.686114 4.823236)
    (xy -42.704216 4.480449) (xy -42.719107 4.0706) (xy -42.73073 3.607879) (xy -42.739031 3.106475) (xy -42.743955 2.580576)
    (xy -42.745446 2.04437) (xy -42.743449 1.512047) (xy -42.737909 0.997795) (xy -42.728771 0.515802) (xy -42.71598 0.080258)
    (xy -42.699479 -0.294648) (xy -42.686579 -0.501316) (xy -42.640677 -1.073023) (xy -42.584504 -1.672099) (xy -42.520166 -2.281538)
    (xy -42.449767 -2.884333) (xy -42.375411 -3.463477) (xy -42.299202 -4.001964) (xy -42.223245 -4.482785) (xy -42.149644 -4.888935)
    (xy -42.134218 -4.965414) (xy -42.103709 -5.116356) (xy -42.061815 -5.327557) (xy -42.01516 -5.5655) (xy -41.987968 -5.705452)
    (xy -41.917812 -6.044279) (xy -41.825531 -6.454319) (xy -41.71628 -6.915275) (xy -41.595213 -7.406849) (xy -41.467484 -7.908744)
    (xy -41.338248 -8.400664) (xy -41.212659 -8.862312) (xy -41.095872 -9.27339) (xy -41.00586 -9.572745) (xy -40.875635 -9.984265)
    (xy -40.737268 -10.410441) (xy -40.596657 -10.833923) (xy -40.459699 -11.237361) (xy -40.332291 -11.603405) (xy -40.220331 -11.914706)
    (xy -40.129715 -12.153913) (xy -40.12141 -12.174813) (xy -40.036751 -12.387914) (xy -39.960458 -12.58236) (xy -39.902697 -12.732114)
    (xy -39.879064 -12.795489) (xy -39.826303 -12.932138) (xy -39.758467 -13.095589) (xy -39.739457 -13.139423) (xy -39.689297 -13.264627)
    (xy -39.675665 -13.357741) (xy -39.698101 -13.463504) (xy -39.73506 -13.569122) (xy -39.753269 -13.625205) (xy -39.768569 -13.690911)
    (xy -39.781166 -13.774308) (xy -39.791264 -13.883466) (xy -39.79907 -14.026453) (xy -39.804789 -14.21134) (xy -39.808626 -14.446194)
    (xy -39.810787 -14.739086) (xy -39.811477 -15.098083) (xy -39.810902 -15.531256) (xy -39.809268 -16.046674) (xy -39.807757 -16.424061)
    (xy -39.804035 -17.071941) (xy -39.798671 -17.643839) (xy -39.791734 -18.136704) (xy -39.783291 -18.547488) (xy -39.77341 -18.873139)
    (xy -39.762158 -19.11061) (xy -39.749602 -19.256849) (xy -39.744318 -19.288722) (xy -39.718213 -19.438327) (xy -39.693033 -19.647683)
    (xy -39.668382 -19.92253) (xy -39.643862 -20.268605) (xy -39.619077 -20.691646) (xy -39.593628 -21.197392) (xy -39.567119 -21.791581)
    (xy -39.560948 -21.938534) (xy -39.517786 -22.936258) (xy -39.474743 -23.846347) (xy -39.431257 -24.67665) (xy -39.386765 -25.435019)
    (xy -39.340705 -26.129304) (xy -39.292515 -26.767356) (xy -39.241634 -27.357026) (xy -39.187497 -27.906165) (xy -39.129545 -28.422622)
    (xy -39.067213 -28.914249) (xy -39.054938 -29.0047) (xy -38.977002 -29.565221) (xy -38.908125 -30.04101) (xy -38.846316 -30.442183)
    (xy -38.789584 -30.778853) (xy -38.735935 -31.061137) (xy -38.68338 -31.299149) (xy -38.629926 -31.503005) (xy -38.573581 -31.682819)
    (xy -38.512355 -31.848707) (xy -38.478798 -31.930753) (xy -38.410727 -32.097905) (xy -38.356438 -32.241169) (xy -38.329631 -32.322933)
    (xy -38.295111 -32.403601) (xy -38.222196 -32.542166) (xy -38.1233 -32.715678) (xy -38.059465 -32.822402) (xy -37.863829 -33.111204)
    (xy -37.668211 -33.32915) (xy -37.550941 -33.429208) (xy -37.415344 -33.530626) (xy -37.309089 -33.603989) (xy -37.25452 -33.633899)
    (xy -37.253844 -33.633968) (xy -37.195206 -33.654017) (xy -37.078628 -33.703988) (xy -36.962921 -33.757312) (xy -36.870243 -33.79961)
    (xy -36.786242 -33.830457) (xy -36.694495 -33.851361) (xy -36.578578 -33.863832) (xy -36.422069 -33.86938) (xy -36.208545 -33.869512))
   (stroke (width 0.5) (type solid)) (fill no) (layer "Edge.Cuts")))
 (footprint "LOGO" (layer "F.Cu") (at 131 108)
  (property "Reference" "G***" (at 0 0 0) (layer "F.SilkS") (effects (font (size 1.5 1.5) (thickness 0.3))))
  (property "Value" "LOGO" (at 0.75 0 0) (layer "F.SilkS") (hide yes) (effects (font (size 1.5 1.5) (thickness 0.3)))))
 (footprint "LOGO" (layer "F.Cu") (at 161 78 -10)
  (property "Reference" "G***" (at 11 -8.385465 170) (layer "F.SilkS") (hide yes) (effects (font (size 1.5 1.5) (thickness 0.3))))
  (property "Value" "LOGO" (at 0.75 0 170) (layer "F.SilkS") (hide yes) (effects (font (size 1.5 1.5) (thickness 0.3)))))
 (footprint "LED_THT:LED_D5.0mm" (layer "F.Cu") (at 119.581103 88.75)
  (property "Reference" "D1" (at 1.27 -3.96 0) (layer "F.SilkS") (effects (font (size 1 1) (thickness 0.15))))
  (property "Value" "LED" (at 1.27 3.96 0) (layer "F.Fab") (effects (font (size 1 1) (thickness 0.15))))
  (pad "1" thru_hole rect (at 0 0) (size 1.8 1.8) (drill 0.9) (layers "*.Cu" "*.Mask") (remove_unused_layers no) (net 1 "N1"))
  (pad "2" thru_hole circle (at 2.54 0) (size 1.8 1.8) (drill 0.9) (layers "*.Cu" "*.Mask") (remove_unused_layers no) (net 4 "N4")))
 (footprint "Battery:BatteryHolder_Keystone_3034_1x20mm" (layer "B.Cu") (at 130.5 100.5)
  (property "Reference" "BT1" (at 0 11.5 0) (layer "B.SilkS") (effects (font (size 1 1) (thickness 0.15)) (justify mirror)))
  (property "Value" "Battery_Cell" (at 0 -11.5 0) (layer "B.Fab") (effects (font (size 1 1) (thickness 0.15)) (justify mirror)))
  (pad "1" smd rect (at -10.985 0) (size 1.27 5.08) (layers "B.Cu" "B.Mask" "B.Paste") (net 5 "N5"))
  (pad "1" smd rect (at 10.985 0) (size 1.27 5.08) (layers "B.Cu" "B.Mask" "B.Paste") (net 5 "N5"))
  (pad "2" smd circle (at 0 0) (size 17.8 17.8) (layers "B.Cu" "B.Mask") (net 3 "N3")))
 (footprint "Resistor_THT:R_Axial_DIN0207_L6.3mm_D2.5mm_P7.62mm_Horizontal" (layer "B.Cu") (at 139.391103 112.75 180)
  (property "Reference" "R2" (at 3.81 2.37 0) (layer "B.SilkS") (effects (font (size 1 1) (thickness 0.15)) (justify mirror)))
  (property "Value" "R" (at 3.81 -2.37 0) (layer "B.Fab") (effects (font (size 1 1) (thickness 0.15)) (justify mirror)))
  (pad "1" thru_hole circle (at 0 0 180) (size 1.6 1.6) (drill 0.8) (layers "*.Cu" "*.Mask") (remove_unused_layers no) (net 5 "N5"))
  (pad "2" thru_hole circle (at 7.62 0 180) (size 1.6 1.6) (drill 0.8) (layers "*.Cu" "*.Mask") (remove_unused_layers no) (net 2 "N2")))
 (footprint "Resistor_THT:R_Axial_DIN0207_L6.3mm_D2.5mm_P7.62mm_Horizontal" (layer "B.Cu") (at 129.391103 112.75 180)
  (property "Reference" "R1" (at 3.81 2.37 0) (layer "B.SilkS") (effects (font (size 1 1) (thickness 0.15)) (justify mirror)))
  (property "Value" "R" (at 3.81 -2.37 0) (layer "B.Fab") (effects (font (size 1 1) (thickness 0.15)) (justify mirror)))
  (pad "1" thru_hole circle (at 0 0 180) (size 1.6 1.6) (drill 0.8) (layers "*.Cu" "*.Mask") (remove_unused_layers no) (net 5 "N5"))
  (pad "2" thru_hole circle (at 7.62 0 180) (size 1.6 1.6) (drill 0.8) (layers "*.Cu" "*.Mask") (remove_unused_layers no) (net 4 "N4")))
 (via (at 131 77) (size 5.5) (drill 5) (layers "F.Cu" "B.Cu") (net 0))
 (segment (start 129.391103 112.75) (end 130.492103 113.851) (width 0.2) (layer "F.Cu") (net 5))
 (segment (start 138.290103 113.851) (end 139.391103 112.75) (width 0.2) (layer "F.Cu") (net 5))
 (segment (start 130.492103 113.851) (end 138.290103 113.851) (width 0.2) (layer "F.Cu") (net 5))
 (segment (start 119.515 100.5) (end 119.515 108.936847) (width 0.2) (layer "B.Cu") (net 5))
 (segment (start 141.485 110.656103) (end 141.485 100.5) (width 0.2) (layer "B.Cu") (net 5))
 (segment (start 139.391103 112.75) (end 141.485 110.656103) (width 0.2) (layer "B.Cu") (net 5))
 (segment (start 119.515 108.936847) (end 123.328153 112.75) (width 0.2) (layer "B.Cu") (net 5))
 (segment (start 123.328153 112.75) (end 129.391103 112.75) (width 0.2) (layer "B.Cu") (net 5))
 (segment (start 120.920103 87.549) (end 118.380103 87.549) (width 0.2) (layer "F.Cu") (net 4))
 (segment (start 122.121103 88.75) (end 120.920103 87.549) (width 0.2) (layer "F.Cu") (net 4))
 (segment (start 118.380103 87.549) (end 118.380103 109.359) (width 0.2) (layer "F.Cu") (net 4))
 (segment (start 118.380103 109.359) (end 121.771103 112.75) (width 0.2) (layer "F.Cu") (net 4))
 (segment (start 127.081103 99.75) (end 119.581103 92.25) (width 0.2) (layer "F.Cu") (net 1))
 (segment (start 133.581103 99.75) (end 127.081103 99.75) (width 0.2) (layer "F.Cu") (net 1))
 (segment (start 139.041103 94.29) (end 133.581103 99.75) (width 0.2) (layer "F.Cu") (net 1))
 (segment (start 139.041103 88.75) (end 139.041103 94.29) (width 0.2) (layer "F.Cu") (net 1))
 (segment (start 119.581103 92.25) (end 119.581103 88.75) (width 0.2) (layer "F.Cu") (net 1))
 (segment (start 139.041103 88.75) (end 139.782103 89.491) (width 0.2) (layer "B.Cu") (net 1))
 (segment (start 141.581103 102.94) (end 131.771103 112.75) (width 0.2) (layer "F.Cu") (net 2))
 (segment (start 141.581103 88.75) (end 141.581103 102.94) (width 0.2) (layer "F.Cu") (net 2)))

